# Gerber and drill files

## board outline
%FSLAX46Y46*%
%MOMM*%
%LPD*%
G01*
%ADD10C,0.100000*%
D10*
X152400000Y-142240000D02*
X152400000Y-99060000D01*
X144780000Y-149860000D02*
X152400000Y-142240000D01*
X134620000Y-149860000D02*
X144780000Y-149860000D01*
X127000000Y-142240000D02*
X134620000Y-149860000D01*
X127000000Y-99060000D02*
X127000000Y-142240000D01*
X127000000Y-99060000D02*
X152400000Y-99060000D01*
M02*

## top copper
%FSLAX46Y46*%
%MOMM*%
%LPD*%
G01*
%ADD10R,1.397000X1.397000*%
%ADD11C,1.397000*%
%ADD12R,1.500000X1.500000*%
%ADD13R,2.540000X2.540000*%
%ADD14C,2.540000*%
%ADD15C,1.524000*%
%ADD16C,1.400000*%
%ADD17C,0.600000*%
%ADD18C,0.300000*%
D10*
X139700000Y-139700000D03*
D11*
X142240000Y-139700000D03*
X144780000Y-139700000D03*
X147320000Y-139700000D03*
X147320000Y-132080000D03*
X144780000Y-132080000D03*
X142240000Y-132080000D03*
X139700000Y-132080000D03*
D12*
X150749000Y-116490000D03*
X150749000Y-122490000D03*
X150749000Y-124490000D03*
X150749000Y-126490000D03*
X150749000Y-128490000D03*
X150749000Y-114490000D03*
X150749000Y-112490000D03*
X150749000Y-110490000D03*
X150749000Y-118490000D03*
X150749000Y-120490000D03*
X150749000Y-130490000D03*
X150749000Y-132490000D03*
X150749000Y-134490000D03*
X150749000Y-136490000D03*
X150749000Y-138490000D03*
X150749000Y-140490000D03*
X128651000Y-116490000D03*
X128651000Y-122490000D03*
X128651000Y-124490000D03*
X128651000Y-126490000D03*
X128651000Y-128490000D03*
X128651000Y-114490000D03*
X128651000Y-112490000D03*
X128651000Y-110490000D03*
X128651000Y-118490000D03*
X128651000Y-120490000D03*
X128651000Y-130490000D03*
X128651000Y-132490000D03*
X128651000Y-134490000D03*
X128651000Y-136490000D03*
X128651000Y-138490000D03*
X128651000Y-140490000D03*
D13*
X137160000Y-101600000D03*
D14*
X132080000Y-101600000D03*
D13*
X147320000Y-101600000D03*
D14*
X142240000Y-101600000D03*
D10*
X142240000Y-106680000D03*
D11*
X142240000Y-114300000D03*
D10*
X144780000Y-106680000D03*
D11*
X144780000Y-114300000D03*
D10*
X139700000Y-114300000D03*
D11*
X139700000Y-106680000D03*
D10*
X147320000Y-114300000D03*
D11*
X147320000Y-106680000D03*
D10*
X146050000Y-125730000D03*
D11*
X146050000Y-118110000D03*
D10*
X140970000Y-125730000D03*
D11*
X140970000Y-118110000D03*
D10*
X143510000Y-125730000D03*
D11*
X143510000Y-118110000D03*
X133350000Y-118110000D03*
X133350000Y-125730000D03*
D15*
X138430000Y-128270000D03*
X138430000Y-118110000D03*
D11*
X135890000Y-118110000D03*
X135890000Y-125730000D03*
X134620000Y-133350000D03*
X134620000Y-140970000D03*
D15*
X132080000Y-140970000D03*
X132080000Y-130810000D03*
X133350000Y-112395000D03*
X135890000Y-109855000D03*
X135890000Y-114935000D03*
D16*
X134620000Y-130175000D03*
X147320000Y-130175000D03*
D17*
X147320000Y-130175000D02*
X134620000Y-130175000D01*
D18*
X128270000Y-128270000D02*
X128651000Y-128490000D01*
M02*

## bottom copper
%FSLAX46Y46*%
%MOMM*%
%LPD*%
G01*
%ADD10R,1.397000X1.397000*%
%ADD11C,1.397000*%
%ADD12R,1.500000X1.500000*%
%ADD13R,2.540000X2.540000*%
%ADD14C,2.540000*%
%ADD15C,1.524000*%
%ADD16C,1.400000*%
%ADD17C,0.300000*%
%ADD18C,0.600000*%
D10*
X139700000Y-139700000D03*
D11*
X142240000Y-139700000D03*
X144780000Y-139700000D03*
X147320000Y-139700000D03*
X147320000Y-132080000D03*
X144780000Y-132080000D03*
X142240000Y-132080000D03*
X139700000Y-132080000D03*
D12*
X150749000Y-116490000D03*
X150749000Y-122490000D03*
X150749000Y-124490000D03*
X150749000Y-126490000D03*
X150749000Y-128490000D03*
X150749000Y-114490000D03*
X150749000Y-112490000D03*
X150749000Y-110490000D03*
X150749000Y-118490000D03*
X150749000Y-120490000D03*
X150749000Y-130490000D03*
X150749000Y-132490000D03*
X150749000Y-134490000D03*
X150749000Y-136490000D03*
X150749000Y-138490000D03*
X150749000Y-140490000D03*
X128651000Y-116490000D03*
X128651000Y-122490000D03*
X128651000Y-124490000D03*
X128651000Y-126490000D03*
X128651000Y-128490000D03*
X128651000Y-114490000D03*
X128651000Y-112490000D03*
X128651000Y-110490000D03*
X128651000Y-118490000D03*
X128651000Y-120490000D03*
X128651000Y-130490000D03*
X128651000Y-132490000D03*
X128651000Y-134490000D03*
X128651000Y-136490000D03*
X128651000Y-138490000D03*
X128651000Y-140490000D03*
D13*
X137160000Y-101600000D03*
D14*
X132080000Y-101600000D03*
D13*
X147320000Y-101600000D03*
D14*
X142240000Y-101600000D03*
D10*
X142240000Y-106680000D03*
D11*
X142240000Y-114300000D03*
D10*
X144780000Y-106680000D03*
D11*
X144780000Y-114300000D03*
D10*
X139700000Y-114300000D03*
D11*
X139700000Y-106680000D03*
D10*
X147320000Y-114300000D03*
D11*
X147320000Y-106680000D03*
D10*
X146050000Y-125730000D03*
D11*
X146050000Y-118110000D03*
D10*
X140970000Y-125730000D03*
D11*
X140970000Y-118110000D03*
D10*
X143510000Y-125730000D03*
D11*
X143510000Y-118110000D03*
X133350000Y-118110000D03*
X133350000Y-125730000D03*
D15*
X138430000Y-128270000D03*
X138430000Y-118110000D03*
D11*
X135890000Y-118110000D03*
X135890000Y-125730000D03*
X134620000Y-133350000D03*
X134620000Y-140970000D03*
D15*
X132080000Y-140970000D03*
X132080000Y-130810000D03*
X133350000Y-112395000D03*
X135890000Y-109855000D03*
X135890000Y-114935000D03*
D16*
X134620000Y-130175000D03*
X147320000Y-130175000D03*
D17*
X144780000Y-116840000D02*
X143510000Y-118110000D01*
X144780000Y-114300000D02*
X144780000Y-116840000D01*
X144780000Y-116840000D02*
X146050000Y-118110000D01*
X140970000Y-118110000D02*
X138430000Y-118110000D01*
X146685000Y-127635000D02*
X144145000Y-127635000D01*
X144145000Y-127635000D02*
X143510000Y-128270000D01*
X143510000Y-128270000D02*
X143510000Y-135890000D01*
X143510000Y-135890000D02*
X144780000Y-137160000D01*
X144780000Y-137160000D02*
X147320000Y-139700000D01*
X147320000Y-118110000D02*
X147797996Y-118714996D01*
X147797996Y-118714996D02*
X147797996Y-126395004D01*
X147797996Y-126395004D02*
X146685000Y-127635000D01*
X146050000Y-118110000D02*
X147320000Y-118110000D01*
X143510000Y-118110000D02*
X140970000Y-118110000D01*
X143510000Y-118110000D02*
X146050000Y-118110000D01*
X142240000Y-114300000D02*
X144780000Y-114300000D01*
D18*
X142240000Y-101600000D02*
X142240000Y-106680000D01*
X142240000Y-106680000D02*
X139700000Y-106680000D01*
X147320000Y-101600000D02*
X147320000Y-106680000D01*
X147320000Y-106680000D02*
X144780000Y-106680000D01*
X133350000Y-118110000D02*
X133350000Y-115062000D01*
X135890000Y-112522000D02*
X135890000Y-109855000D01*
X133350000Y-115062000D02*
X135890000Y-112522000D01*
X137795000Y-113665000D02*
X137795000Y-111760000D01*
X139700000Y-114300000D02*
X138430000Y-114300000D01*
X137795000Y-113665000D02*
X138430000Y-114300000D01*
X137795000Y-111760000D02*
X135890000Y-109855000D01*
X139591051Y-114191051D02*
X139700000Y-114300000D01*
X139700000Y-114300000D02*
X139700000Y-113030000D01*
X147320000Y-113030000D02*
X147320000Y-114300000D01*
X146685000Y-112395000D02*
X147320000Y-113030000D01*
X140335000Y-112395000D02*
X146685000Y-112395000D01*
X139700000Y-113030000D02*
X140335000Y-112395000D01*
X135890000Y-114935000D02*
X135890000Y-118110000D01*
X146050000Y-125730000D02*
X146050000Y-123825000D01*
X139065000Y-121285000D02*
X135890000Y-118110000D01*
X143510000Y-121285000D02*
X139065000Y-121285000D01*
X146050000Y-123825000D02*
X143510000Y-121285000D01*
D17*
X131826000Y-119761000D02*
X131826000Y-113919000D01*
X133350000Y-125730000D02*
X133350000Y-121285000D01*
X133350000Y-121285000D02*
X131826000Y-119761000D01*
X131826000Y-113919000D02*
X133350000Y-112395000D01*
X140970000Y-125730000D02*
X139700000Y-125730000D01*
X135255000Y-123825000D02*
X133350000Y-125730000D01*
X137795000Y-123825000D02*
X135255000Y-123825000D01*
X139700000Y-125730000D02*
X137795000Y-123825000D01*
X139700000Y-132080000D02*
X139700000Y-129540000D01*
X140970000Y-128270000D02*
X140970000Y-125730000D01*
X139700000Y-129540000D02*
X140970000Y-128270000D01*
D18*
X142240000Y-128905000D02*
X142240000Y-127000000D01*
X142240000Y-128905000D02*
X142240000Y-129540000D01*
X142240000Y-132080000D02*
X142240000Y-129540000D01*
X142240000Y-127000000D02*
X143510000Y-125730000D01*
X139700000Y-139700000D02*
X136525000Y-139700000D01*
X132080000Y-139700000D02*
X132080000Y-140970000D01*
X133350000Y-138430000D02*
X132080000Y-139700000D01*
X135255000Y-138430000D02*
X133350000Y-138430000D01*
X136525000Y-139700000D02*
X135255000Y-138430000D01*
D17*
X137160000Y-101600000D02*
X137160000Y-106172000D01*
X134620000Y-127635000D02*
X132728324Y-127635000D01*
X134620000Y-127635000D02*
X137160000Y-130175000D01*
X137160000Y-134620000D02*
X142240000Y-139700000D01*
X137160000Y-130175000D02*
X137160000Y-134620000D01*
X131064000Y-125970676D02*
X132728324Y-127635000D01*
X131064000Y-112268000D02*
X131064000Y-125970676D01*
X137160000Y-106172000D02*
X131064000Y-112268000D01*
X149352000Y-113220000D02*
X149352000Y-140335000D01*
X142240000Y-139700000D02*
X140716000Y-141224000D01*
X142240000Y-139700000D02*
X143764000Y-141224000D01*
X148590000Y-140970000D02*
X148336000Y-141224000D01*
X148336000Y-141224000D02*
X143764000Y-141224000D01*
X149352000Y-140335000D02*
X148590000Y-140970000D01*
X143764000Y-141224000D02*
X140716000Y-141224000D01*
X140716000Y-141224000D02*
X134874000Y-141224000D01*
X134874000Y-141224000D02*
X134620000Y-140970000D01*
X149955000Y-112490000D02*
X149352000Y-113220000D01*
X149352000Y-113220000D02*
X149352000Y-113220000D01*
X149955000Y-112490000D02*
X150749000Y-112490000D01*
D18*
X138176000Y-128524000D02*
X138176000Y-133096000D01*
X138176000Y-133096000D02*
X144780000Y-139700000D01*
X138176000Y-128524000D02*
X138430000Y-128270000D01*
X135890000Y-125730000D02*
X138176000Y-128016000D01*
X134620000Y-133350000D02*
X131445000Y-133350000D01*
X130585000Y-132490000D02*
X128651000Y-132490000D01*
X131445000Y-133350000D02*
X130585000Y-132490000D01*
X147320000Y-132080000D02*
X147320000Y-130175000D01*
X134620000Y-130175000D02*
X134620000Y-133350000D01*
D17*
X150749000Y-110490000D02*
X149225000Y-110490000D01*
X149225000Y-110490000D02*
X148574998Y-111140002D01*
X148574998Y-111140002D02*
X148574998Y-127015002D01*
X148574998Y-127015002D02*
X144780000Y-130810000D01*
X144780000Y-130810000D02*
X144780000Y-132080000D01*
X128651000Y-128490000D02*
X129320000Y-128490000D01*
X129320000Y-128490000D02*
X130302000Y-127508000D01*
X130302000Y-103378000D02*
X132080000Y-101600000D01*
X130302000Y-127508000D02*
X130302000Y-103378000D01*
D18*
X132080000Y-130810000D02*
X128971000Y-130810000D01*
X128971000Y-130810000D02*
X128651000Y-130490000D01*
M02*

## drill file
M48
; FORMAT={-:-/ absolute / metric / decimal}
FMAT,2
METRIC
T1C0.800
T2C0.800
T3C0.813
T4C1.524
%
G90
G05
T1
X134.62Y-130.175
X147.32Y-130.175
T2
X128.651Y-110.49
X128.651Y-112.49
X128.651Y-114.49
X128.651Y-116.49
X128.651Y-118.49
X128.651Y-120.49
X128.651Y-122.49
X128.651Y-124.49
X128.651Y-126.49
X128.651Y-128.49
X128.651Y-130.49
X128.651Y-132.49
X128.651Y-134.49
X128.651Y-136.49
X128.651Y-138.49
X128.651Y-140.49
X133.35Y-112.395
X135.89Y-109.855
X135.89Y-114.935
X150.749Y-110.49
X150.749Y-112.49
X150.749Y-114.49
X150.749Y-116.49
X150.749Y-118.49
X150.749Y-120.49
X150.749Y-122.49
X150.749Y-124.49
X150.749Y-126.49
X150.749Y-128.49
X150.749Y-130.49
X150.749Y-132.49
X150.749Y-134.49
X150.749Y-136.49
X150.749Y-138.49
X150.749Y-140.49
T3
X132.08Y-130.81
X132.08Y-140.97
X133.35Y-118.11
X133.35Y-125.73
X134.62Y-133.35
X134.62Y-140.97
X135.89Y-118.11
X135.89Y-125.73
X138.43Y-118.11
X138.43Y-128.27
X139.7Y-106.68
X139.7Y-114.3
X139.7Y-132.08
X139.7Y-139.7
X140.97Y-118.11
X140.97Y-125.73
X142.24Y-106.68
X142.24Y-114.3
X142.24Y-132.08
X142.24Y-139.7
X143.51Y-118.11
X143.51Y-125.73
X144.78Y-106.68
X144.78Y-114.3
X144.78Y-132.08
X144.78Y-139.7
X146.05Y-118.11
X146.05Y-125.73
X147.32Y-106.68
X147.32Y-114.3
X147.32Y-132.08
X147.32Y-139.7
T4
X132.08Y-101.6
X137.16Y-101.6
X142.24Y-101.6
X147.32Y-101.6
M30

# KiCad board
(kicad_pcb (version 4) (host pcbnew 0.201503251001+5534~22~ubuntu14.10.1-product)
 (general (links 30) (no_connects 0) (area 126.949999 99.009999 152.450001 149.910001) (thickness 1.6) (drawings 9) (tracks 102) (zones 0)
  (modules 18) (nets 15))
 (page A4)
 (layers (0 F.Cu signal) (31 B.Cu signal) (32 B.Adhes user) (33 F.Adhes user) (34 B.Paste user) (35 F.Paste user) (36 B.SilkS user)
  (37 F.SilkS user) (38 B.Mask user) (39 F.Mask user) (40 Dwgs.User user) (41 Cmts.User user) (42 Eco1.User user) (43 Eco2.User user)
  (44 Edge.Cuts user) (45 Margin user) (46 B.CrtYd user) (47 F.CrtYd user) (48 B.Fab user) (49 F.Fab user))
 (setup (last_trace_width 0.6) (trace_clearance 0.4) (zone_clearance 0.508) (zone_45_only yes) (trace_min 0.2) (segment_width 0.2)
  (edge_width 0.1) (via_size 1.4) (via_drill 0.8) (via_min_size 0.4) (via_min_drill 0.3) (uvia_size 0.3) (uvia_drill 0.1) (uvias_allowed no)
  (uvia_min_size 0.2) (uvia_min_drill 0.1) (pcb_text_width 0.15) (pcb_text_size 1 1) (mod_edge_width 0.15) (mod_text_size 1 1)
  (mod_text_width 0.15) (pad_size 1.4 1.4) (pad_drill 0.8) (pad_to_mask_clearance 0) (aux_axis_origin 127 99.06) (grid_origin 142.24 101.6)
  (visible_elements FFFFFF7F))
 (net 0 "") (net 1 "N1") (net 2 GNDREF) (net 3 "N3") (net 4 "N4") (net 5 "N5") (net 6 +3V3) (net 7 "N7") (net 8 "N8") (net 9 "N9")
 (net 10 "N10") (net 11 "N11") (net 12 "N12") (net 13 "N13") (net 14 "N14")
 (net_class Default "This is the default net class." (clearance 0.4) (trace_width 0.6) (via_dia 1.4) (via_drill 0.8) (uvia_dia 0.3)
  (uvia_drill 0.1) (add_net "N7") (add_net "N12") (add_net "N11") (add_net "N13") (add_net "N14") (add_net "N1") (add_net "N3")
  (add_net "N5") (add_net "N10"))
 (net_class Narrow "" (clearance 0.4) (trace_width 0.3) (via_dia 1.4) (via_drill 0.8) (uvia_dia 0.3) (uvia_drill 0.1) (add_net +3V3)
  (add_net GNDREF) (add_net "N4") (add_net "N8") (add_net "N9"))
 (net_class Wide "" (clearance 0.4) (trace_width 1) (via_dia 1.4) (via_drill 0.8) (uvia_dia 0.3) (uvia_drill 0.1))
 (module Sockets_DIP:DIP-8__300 (layer F.Cu) (at 143.51 135.89)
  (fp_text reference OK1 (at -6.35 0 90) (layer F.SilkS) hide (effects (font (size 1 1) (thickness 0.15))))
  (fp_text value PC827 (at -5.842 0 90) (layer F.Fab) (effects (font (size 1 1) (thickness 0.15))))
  (pad 1 thru_hole rect (at -3.81 3.81) (size 1.397 1.397) (drill 0.8128) (layers *.Cu *.Mask F.SilkS) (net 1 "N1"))
  (pad 2 thru_hole circle (at -1.27 3.81) (size 1.397 1.397) (drill 0.8128) (layers *.Cu *.Mask F.SilkS) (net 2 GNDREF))
  (pad 3 thru_hole circle (at 1.27 3.81) (size 1.397 1.397) (drill 0.8128) (layers *.Cu *.Mask F.SilkS) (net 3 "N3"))
  (pad 4 thru_hole circle (at 3.81 3.81) (size 1.397 1.397) (drill 0.8128) (layers *.Cu *.Mask F.SilkS) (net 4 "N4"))
  (pad 5 thru_hole circle (at 3.81 -3.81) (size 1.397 1.397) (drill 0.8128) (layers *.Cu *.Mask F.SilkS) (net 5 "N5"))
  (pad 6 thru_hole circle (at 1.27 -3.81) (size 1.397 1.397) (drill 0.8128) (layers *.Cu *.Mask F.SilkS) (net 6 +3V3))
  (pad 7 thru_hole circle (at -1.27 -3.81) (size 1.397 1.397) (drill 0.8128) (layers *.Cu *.Mask F.SilkS) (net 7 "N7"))
  (pad 8 thru_hole circle (at -3.81 -3.81) (size 1.397 1.397) (drill 0.8128) (layers *.Cu *.Mask F.SilkS) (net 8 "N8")))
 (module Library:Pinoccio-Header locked (layer F.Cu) (at 150.749 125.49)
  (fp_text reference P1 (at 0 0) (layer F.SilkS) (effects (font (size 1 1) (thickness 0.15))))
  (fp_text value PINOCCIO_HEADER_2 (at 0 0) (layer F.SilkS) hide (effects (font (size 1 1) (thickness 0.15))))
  (pad 4 thru_hole rect (at 0 -9) (size 1.5 1.5) (drill 0.8) (layers *.Cu *.Mask F.SilkS))
  (pad 7 thru_hole rect (at 0 -3) (size 1.5 1.5) (drill 0.8) (layers *.Cu *.Mask F.SilkS))
  (pad 8 thru_hole rect (at 0 -1) (size 1.5 1.5) (drill 0.8) (layers *.Cu *.Mask F.SilkS))
  (pad 9 thru_hole rect (at 0 1) (size 1.5 1.5) (drill 0.8) (layers *.Cu *.Mask F.SilkS))
  (pad 10 thru_hole rect (at 0 3) (size 1.5 1.5) (drill 0.8) (layers *.Cu *.Mask F.SilkS))
  (pad 3 thru_hole rect (at 0 -11) (size 1.5 1.5) (drill 0.8) (layers *.Cu *.Mask F.SilkS))
  (pad 2 thru_hole rect (at 0 -13) (size 1.5 1.5) (drill 0.8) (layers *.Cu *.Mask F.SilkS) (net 2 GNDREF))
  (pad 1 thru_hole rect (at 0 -15) (size 1.5 1.5) (drill 0.8) (layers *.Cu *.Mask F.SilkS) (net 6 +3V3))
  (pad 5 thru_hole rect (at 0 -7) (size 1.5 1.5) (drill 0.8) (layers *.Cu *.Mask F.SilkS))
  (pad 6 thru_hole rect (at 0 -5) (size 1.5 1.5) (drill 0.8) (layers *.Cu *.Mask F.SilkS))
  (pad 11 thru_hole rect (at 0 5) (size 1.5 1.5) (drill 0.8) (layers *.Cu *.Mask F.SilkS))
  (pad 12 thru_hole rect (at 0 7) (size 1.5 1.5) (drill 0.8) (layers *.Cu *.Mask F.SilkS))
  (pad 13 thru_hole rect (at 0 9) (size 1.5 1.5) (drill 0.8) (layers *.Cu *.Mask F.SilkS))
  (pad 14 thru_hole rect (at 0 11) (size 1.5 1.5) (drill 0.8) (layers *.Cu *.Mask F.SilkS))
  (pad 15 thru_hole rect (at 0 13) (size 1.5 1.5) (drill 0.8) (layers *.Cu *.Mask F.SilkS))
  (pad 16 thru_hole rect (at 0 15) (size 1.5 1.5) (drill 0.8) (layers *.Cu *.Mask F.SilkS)))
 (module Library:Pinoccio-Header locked (layer F.Cu) (at 128.651 125.49)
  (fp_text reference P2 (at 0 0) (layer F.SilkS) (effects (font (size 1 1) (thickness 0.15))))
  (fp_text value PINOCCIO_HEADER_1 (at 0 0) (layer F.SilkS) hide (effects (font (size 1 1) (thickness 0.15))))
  (pad 4 thru_hole rect (at 0 -9) (size 1.5 1.5) (drill 0.8) (layers *.Cu *.Mask F.SilkS))
  (pad 7 thru_hole rect (at 0 -3) (size 1.5 1.5) (drill 0.8) (layers *.Cu *.Mask F.SilkS))
  (pad 8 thru_hole rect (at 0 -1) (size 1.5 1.5) (drill 0.8) (layers *.Cu *.Mask F.SilkS))
  (pad 9 thru_hole rect (at 0 1) (size 1.5 1.5) (drill 0.8) (layers *.Cu *.Mask F.SilkS))
  (pad 10 thru_hole rect (at 0 3) (size 1.5 1.5) (drill 0.8) (layers *.Cu *.Mask F.SilkS) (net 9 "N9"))
  (pad 3 thru_hole rect (at 0 -11) (size 1.5 1.5) (drill 0.8) (layers *.Cu *.Mask F.SilkS))
  (pad 2 thru_hole rect (at 0 -13) (size 1.5 1.5) (drill 0.8) (layers *.Cu *.Mask F.SilkS))
  (pad 1 thru_hole rect (at 0 -15) (size 1.5 1.5) (drill 0.8) (layers *.Cu *.Mask F.SilkS))
  (pad 5 thru_hole rect (at 0 -7) (size 1.5 1.5) (drill 0.8) (layers *.Cu *.Mask F.SilkS))
  (pad 6 thru_hole rect (at 0 -5) (size 1.5 1.5) (drill 0.8) (layers *.Cu *.Mask F.SilkS))
  (pad 11 thru_hole rect (at 0 5) (size 1.5 1.5) (drill 0.8) (layers *.Cu *.Mask F.SilkS) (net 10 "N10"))
  (pad 12 thru_hole rect (at 0 7) (size 1.5 1.5) (drill 0.8) (layers *.Cu *.Mask F.SilkS) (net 5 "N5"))
  (pad 13 thru_hole rect (at 0 9) (size 1.5 1.5) (drill 0.8) (layers *.Cu *.Mask F.SilkS))
  (pad 14 thru_hole rect (at 0 11) (size 1.5 1.5) (drill 0.8) (layers *.Cu *.Mask F.SilkS))
  (pad 15 thru_hole rect (at 0 13) (size 1.5 1.5) (drill 0.8) (layers *.Cu *.Mask F.SilkS))
  (pad 16 thru_hole rect (at 0 15) (size 1.5 1.5) (drill 0.8) (layers *.Cu *.Mask F.SilkS)))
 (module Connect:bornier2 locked (layer F.Cu) (at 134.62 101.6 180)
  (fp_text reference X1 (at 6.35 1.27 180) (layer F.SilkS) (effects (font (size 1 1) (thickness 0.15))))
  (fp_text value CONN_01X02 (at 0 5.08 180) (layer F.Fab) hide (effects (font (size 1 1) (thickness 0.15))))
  (pad 1 thru_hole rect (at -2.54 0 180) (size 2.54 2.54) (drill 1.524) (layers *.Cu *.Mask F.SilkS) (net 2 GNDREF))
  (pad 2 thru_hole circle (at 2.54 0 180) (size 2.54 2.54) (drill 1.524) (layers *.Cu *.Mask F.SilkS) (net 9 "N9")))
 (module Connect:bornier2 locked (layer F.Cu) (at 144.78 101.6 180)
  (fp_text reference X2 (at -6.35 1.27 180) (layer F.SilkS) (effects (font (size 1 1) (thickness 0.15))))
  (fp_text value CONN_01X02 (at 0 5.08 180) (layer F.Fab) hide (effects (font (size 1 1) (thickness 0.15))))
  (pad 1 thru_hole rect (at -2.54 0 180) (size 2.54 2.54) (drill 1.524) (layers *.Cu *.Mask F.SilkS) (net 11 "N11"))
  (pad 2 thru_hole circle (at 2.54 0 180) (size 2.54 2.54) (drill 1.524) (layers *.Cu *.Mask F.SilkS) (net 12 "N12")))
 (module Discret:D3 (layer F.Cu) (at 142.24 110.49 90)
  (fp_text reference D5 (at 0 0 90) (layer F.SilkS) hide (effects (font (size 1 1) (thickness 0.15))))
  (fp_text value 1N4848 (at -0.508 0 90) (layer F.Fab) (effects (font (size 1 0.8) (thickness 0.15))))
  (pad 2 thru_hole rect (at 3.81 0 90) (size 1.397 1.397) (drill 0.8128) (layers *.Cu *.Mask F.SilkS) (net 12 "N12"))
  (pad 1 thru_hole circle (at -3.81 0 90) (size 1.397 1.397) (drill 0.8128) (layers *.Cu *.Mask F.SilkS) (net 4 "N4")))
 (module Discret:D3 (layer F.Cu) (at 144.78 110.49 90)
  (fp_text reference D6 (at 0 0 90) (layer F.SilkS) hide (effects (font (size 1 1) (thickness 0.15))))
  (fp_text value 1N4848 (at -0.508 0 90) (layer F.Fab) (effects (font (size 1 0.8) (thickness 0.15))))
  (pad 2 thru_hole rect (at 3.81 0 90) (size 1.397 1.397) (drill 0.8128) (layers *.Cu *.Mask F.SilkS) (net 11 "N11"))
  (pad 1 thru_hole circle (at -3.81 0 90) (size 1.397 1.397) (drill 0.8128) (layers *.Cu *.Mask F.SilkS) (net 4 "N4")))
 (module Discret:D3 (layer F.Cu) (at 139.7 110.49 270)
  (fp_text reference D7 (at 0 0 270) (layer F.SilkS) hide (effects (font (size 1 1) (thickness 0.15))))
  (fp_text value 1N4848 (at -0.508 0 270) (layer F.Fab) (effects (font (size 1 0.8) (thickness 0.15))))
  (pad 2 thru_hole rect (at 3.81 0 270) (size 1.397 1.397) (drill 0.8128) (layers *.Cu *.Mask F.SilkS) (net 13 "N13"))
  (pad 1 thru_hole circle (at -3.81 0 270) (size 1.397 1.397) (drill 0.8128) (layers *.Cu *.Mask F.SilkS) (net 12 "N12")))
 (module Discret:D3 (layer F.Cu) (at 147.32 110.49 270)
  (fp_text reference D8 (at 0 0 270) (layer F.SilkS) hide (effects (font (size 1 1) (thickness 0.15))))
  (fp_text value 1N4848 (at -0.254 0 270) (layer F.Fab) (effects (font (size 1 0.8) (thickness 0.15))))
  (pad 2 thru_hole rect (at 3.81 0 270) (size 1.397 1.397) (drill 0.8128) (layers *.Cu *.Mask F.SilkS) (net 13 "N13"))
  (pad 1 thru_hole circle (at -3.81 0 270) (size 1.397 1.397) (drill 0.8128) (layers *.Cu *.Mask F.SilkS) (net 11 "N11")))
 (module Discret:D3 (layer F.Cu) (at 146.05 121.92 270)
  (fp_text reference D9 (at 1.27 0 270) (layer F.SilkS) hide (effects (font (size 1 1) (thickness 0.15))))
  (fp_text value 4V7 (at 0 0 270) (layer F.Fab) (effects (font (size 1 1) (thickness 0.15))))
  (pad 2 thru_hole rect (at 3.81 0 270) (size 1.397 1.397) (drill 0.8128) (layers *.Cu *.Mask F.SilkS) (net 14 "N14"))
  (pad 1 thru_hole circle (at -3.81 0 270) (size 1.397 1.397) (drill 0.8128) (layers *.Cu *.Mask F.SilkS) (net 4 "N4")))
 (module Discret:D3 (layer F.Cu) (at 140.97 121.92 270)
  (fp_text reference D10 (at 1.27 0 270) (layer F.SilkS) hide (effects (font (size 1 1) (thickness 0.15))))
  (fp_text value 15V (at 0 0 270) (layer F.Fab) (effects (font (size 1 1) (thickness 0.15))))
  (pad 2 thru_hole rect (at 3.81 0 270) (size 1.397 1.397) (drill 0.8128) (layers *.Cu *.Mask F.SilkS) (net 8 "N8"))
  (pad 1 thru_hole circle (at -3.81 0 270) (size 1.397 1.397) (drill 0.8128) (layers *.Cu *.Mask F.SilkS) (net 4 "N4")))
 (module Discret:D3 (layer F.Cu) (at 143.51 121.92 270)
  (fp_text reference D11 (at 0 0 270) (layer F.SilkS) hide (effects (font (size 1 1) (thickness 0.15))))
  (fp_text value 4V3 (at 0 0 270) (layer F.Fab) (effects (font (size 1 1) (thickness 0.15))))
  (pad 2 thru_hole rect (at 3.81 0 270) (size 1.397 1.397) (drill 0.8128) (layers *.Cu *.Mask F.SilkS) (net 7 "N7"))
  (pad 1 thru_hole circle (at -3.81 0 270) (size 1.397 1.397) (drill 0.8128) (layers *.Cu *.Mask F.SilkS) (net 4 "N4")))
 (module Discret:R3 (layer F.Cu) (at 133.35 121.92 270)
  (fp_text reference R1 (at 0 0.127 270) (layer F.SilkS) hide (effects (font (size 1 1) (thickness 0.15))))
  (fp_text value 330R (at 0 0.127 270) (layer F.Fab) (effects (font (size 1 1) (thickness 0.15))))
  (pad 1 thru_hole circle (at -3.81 0 270) (size 1.397 1.397) (drill 0.8128) (layers *.Cu *.Mask F.SilkS) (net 13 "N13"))
  (pad 2 thru_hole circle (at 3.81 0 270) (size 1.397 1.397) (drill 0.8128) (layers *.Cu *.Mask F.SilkS) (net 8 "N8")))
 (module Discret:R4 (layer F.Cu) (at 138.43 123.19 90)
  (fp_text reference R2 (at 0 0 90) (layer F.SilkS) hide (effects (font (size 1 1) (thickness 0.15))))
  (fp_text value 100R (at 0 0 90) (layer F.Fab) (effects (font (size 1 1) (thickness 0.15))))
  (pad 1 thru_hole circle (at -5.08 0 90) (size 1.524 1.524) (drill 0.8128) (layers *.Cu *.Mask F.SilkS) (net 3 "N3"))
  (pad 2 thru_hole circle (at 5.08 0 90) (size 1.524 1.524) (drill 0.8128) (layers *.Cu *.Mask F.SilkS) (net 4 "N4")))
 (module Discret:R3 (layer F.Cu) (at 135.89 121.92 270)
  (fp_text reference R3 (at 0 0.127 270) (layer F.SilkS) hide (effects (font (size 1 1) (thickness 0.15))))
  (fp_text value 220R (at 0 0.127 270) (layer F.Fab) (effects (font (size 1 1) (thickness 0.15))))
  (pad 1 thru_hole circle (at -3.81 0 270) (size 1.397 1.397) (drill 0.8128) (layers *.Cu *.Mask F.SilkS) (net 14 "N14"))
  (pad 2 thru_hole circle (at 3.81 0 270) (size 1.397 1.397) (drill 0.8128) (layers *.Cu *.Mask F.SilkS) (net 3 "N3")))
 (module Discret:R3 (layer F.Cu) (at 134.62 137.16 270)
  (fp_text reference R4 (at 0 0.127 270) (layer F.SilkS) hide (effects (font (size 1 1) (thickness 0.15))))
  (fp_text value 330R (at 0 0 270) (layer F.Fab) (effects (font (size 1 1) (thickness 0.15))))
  (pad 1 thru_hole circle (at -3.81 0 270) (size 1.397 1.397) (drill 0.8128) (layers *.Cu *.Mask F.SilkS) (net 5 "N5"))
  (pad 2 thru_hole circle (at 3.81 0 270) (size 1.397 1.397) (drill 0.8128) (layers *.Cu *.Mask F.SilkS) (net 2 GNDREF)))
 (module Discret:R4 (layer F.Cu) (at 132.08 135.89 90)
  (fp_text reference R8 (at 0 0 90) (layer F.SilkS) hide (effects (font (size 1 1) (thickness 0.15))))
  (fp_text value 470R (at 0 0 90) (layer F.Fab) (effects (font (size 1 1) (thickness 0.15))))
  (pad 1 thru_hole circle (at -5.08 0 90) (size 1.524 1.524) (drill 0.8128) (layers *.Cu *.Mask F.SilkS) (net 1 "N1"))
  (pad 2 thru_hole circle (at 5.08 0 90) (size 1.524 1.524) (drill 0.8128) (layers *.Cu *.Mask F.SilkS) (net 10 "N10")))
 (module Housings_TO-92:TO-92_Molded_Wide (layer F.Cu) (at 135.89 114.935 90)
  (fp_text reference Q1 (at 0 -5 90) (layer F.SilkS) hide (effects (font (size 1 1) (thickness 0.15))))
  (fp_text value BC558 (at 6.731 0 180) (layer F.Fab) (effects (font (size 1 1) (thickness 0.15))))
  (pad 2 thru_hole circle (at 2.54 -2.54 180) (size 1.524 1.524) (drill 0.8) (layers *.Cu *.Mask F.SilkS) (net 8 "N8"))
  (pad 3 thru_hole circle (at 5.08 0 180) (size 1.524 1.524) (drill 0.8) (layers *.Cu *.Mask F.SilkS) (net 13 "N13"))
  (pad 1 thru_hole circle (at 0 0 180) (size 1.524 1.524) (drill 0.8) (layers *.Cu *.Mask F.SilkS) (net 14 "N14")))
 (gr_line (start 152.4 142.24) (end 152.4 99.06) (angle 90) (layer Edge.Cuts) (width 0.1))
 (gr_line (start 144.78 149.86) (end 152.4 142.24) (angle 90) (layer Edge.Cuts) (width 0.1))
 (gr_line (start 134.62 149.86) (end 144.78 149.86) (angle 90) (layer Edge.Cuts) (width 0.1))
 (gr_line (start 127 142.24) (end 134.62 149.86) (angle 90) (layer Edge.Cuts) (width 0.1))
 (gr_line (start 127 99.06) (end 127 142.24) (angle 90) (layer Edge.Cuts) (width 0.1))
 (gr_line (start 127 99.06) (end 152.4 99.06) (angle 90) (layer Edge.Cuts) (width 0.1))
 (segment (start 144.78 116.84) (end 143.51 118.11) (width 0.3) (layer B.Cu) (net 4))
 (segment (start 144.78 114.3) (end 144.78 116.84) (width 0.3) (layer B.Cu) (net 4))
 (segment (start 144.78 116.84) (end 146.05 118.11) (width 0.3) (layer B.Cu) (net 4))
 (segment (start 140.97 118.11) (end 138.43 118.11) (width 0.3) (layer B.Cu) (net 4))
 (segment (start 146.685 127.635) (end 144.145 127.635) (width 0.3) (layer B.Cu) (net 4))
 (segment (start 144.145 127.635) (end 143.51 128.27) (width 0.3) (layer B.Cu) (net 4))
 (segment (start 143.51 128.27) (end 143.51 135.89) (width 0.3) (layer B.Cu) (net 4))
 (segment (start 143.51 135.89) (end 144.78 137.16) (width 0.3) (layer B.Cu) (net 4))
 (segment (start 144.78 137.16) (end 147.32 139.7) (width 0.3) (layer B.Cu) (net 4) (status 20))
 (segment (start 147.32 118.11) (end 147.797996 118.714996) (width 0.3) (layer B.Cu) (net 4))
 (segment (start 147.797996 118.714996) (end 147.797996 126.395004) (width 0.3) (layer B.Cu) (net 4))
 (segment (start 147.797996 126.395004) (end 146.685 127.635) (width 0.3) (layer B.Cu) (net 4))
 (segment (start 146.05 118.11) (end 147.32 118.11) (width 0.3) (layer B.Cu) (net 4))
 (segment (start 143.51 118.11) (end 140.97 118.11) (width 0.3) (layer B.Cu) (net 4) (status 80010))
 (segment (start 143.51 118.11) (end 146.05 118.11) (width 0.3) (layer B.Cu) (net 4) (status 80020))
 (segment (start 142.24 114.3) (end 144.78 114.3) (width 0.3) (layer B.Cu) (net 4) (status 80020))
 (segment (start 142.24 101.6) (end 142.24 106.68) (width 0.6) (layer B.Cu) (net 12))
 (segment (start 142.24 106.68) (end 139.7 106.68) (width 0.6) (layer B.Cu) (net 12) (status 80010))
 (segment (start 147.32 101.6) (end 147.32 106.68) (width 0.6) (layer B.Cu) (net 11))
 (segment (start 147.32 106.68) (end 144.78 106.68) (width 0.6) (layer B.Cu) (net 11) (status 80010))
 (segment (start 133.35 118.11) (end 133.35 115.062) (width 0.6) (layer B.Cu) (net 13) (status 400000))
 (segment (start 135.89 112.522) (end 135.89 109.855) (width 0.6) (layer B.Cu) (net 13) (status 800000))
 (segment (start 133.35 115.062) (end 135.89 112.522) (width 0.6) (layer B.Cu) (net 13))
 (segment (start 137.795 113.665) (end 137.795 111.76) (width 0.6) (layer B.Cu) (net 13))
 (segment (start 139.7 114.3) (end 138.43 114.3) (width 0.6) (layer B.Cu) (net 13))
 (segment (start 137.795 113.665) (end 138.43 114.3) (width 0.6) (layer B.Cu) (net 13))
 (segment (start 137.795 111.76) (end 135.89 109.855) (width 0.6) (layer B.Cu) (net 13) (status 800000))
 (segment (start 139.591051 114.191051) (end 139.7 114.3) (width 0.6) (layer B.Cu) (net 13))
 (segment (start 139.7 114.3) (end 139.7 113.03) (width 0.6) (layer B.Cu) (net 13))
 (segment (start 147.32 113.03) (end 147.32 114.3) (width 0.6) (layer B.Cu) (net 13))
 (segment (start 146.685 112.395) (end 147.32 113.03) (width 0.6) (layer B.Cu) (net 13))
 (segment (start 140.335 112.395) (end 146.685 112.395) (width 0.6) (layer B.Cu) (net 13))
 (segment (start 139.7 113.03) (end 140.335 112.395) (width 0.6) (layer B.Cu) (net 13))
 (segment (start 135.89 114.935) (end 135.89 118.11) (width 0.6) (layer B.Cu) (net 14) (status C00000))
 (segment (start 146.05 125.73) (end 146.05 123.825) (width 0.6) (layer B.Cu) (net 14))
 (segment (start 139.065 121.285) (end 135.89 118.11) (width 0.6) (layer B.Cu) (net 14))
 (segment (start 143.51 121.285) (end 139.065 121.285) (width 0.6) (layer B.Cu) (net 14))
 (segment (start 146.05 123.825) (end 143.51 121.285) (width 0.6) (layer B.Cu) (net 14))
 (segment (start 131.826 119.761) (end 131.826 113.919) (width 0.3) (layer B.Cu) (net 8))
 (segment (start 133.35 125.73) (end 133.35 121.285) (width 0.3) (layer B.Cu) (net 8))
 (segment (start 133.35 121.285) (end 131.826 119.761) (width 0.3) (layer B.Cu) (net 8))
 (segment (start 131.826 113.919) (end 133.35 112.395) (width 0.3) (layer B.Cu) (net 8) (status 800000))
 (segment (start 140.97 125.73) (end 139.7 125.73) (width 0.3) (layer B.Cu) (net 8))
 (segment (start 135.255 123.825) (end 133.35 125.73) (width 0.3) (layer B.Cu) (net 8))
 (segment (start 137.795 123.825) (end 135.255 123.825) (width 0.3) (layer B.Cu) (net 8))
 (segment (start 139.7 125.73) (end 137.795 123.825) (width 0.3) (layer B.Cu) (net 8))
 (segment (start 139.7 132.08) (end 139.7 129.54) (width 0.3) (layer B.Cu) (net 8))
 (segment (start 140.97 128.27) (end 140.97 125.73) (width 0.3) (layer B.Cu) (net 8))
 (segment (start 139.7 129.54) (end 140.97 128.27) (width 0.3) (layer B.Cu) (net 8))
 (segment (start 142.24 128.905) (end 142.24 127) (width 0.6) (layer B.Cu) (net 7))
 (segment (start 142.24 128.905) (end 142.24 129.54) (width 0.6) (layer B.Cu) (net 7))
 (segment (start 142.24 132.08) (end 142.24 129.54) (width 0.6) (layer B.Cu) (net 7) (status 20))
 (segment (start 142.24 127) (end 143.51 125.73) (width 0.6) (layer B.Cu) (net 7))
 (segment (start 139.7 139.7) (end 136.525 139.7) (width 0.6) (layer B.Cu) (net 1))
 (segment (start 132.08 139.7) (end 132.08 140.97) (width 0.6) (layer B.Cu) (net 1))
 (segment (start 133.35 138.43) (end 132.08 139.7) (width 0.6) (layer B.Cu) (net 1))
 (segment (start 135.255 138.43) (end 133.35 138.43) (width 0.6) (layer B.Cu) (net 1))
 (segment (start 136.525 139.7) (end 135.255 138.43) (width 0.6) (layer B.Cu) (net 1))
 (segment (start 137.16 101.6) (end 137.16 106.172) (width 0.3) (layer B.Cu) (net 2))
 (segment (start 134.62 127.635) (end 132.728324 127.635) (width 0.3) (layer B.Cu) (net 2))
 (segment (start 134.62 127.635) (end 137.16 130.175) (width 0.3) (layer B.Cu) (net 2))
 (segment (start 137.16 134.62) (end 142.24 139.7) (width 0.3) (layer B.Cu) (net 2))
 (segment (start 137.16 130.175) (end 137.16 134.62) (width 0.3) (layer B.Cu) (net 2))
 (segment (start 131.064 125.970676) (end 132.728324 127.635) (width 0.3) (layer B.Cu) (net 2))
 (segment (start 131.064 112.268) (end 131.064 125.970676) (width 0.3) (layer B.Cu) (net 2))
 (segment (start 137.16 106.172) (end 131.064 112.268) (width 0.3) (layer B.Cu) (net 2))
 (segment (start 149.352 113.22) (end 149.352 140.335) (width 0.3) (layer B.Cu) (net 2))
 (segment (start 142.24 139.7) (end 140.716 141.224) (width 0.3) (layer B.Cu) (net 2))
 (segment (start 142.24 139.7) (end 143.764 141.224) (width 0.3) (layer B.Cu) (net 2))
 (segment (start 148.59 140.97) (end 148.336 141.224) (width 0.3) (layer B.Cu) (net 2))
 (segment (start 148.336 141.224) (end 143.764 141.224) (width 0.3) (layer B.Cu) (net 2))
 (segment (start 149.352 140.335) (end 148.59 140.97) (width 0.3) (layer B.Cu) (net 2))
 (segment (start 143.764 141.224) (end 140.716 141.224) (width 0.3) (layer B.Cu) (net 2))
 (segment (start 140.716 141.224) (end 134.874 141.224) (width 0.3) (layer B.Cu) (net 2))
 (segment (start 134.874 141.224) (end 134.62 140.97) (width 0.3) (layer B.Cu) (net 2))
 (segment (start 149.955 112.49) (end 149.352 113.22) (width 0.3) (layer B.Cu) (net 2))
 (segment (start 149.352 113.22) (end 149.352 113.22) (width 0.3) (layer B.Cu) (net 2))
 (segment (start 149.955 112.49) (end 150.749 112.49) (width 0.3) (layer B.Cu) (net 2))
 (segment (start 138.176 128.524) (end 138.176 133.096) (width 0.6) (layer B.Cu) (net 3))
 (segment (start 138.176 133.096) (end 144.78 139.7) (width 0.6) (layer B.Cu) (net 3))
 (segment (start 138.176 128.524) (end 138.43 128.27) (width 0.6) (layer B.Cu) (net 3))
 (segment (start 135.89 125.73) (end 138.176 128.016) (width 0.6) (layer B.Cu) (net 3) (status 80020))
 (segment (start 134.62 133.35) (end 131.445 133.35) (width 0.6) (layer B.Cu) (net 5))
 (segment (start 130.585 132.49) (end 128.651 132.49) (width 0.6) (layer B.Cu) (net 5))
 (segment (start 131.445 133.35) (end 130.585 132.49) (width 0.6) (layer B.Cu) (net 5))
 (segment (start 147.32 132.08) (end 147.32 130.175) (width 0.6) (layer B.Cu) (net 5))
 (segment (start 134.62 130.175) (end 134.62 133.35) (width 0.6) (layer B.Cu) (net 5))
 (via (at 134.62 130.175) (size 1.4) (layers F.Cu B.Cu) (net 5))
 (segment (start 147.32 130.175) (end 134.62 130.175) (width 0.6) (layer F.Cu) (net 5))
 (via (at 147.32 130.175) (size 1.4) (layers F.Cu B.Cu) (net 5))
 (segment (start 150.749 110.49) (end 149.225 110.49) (width 0.3) (layer B.Cu) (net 6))
 (segment (start 149.225 110.49) (end 148.574998 111.140002) (width 0.3) (layer B.Cu) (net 6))
 (segment (start 148.574998 111.140002) (end 148.574998 127.015002) (width 0.3) (layer B.Cu) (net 6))
 (segment (start 148.574998 127.015002) (end 144.78 130.81) (width 0.3) (layer B.Cu) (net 6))
 (segment (start 144.78 130.81) (end 144.78 132.08) (width 0.3) (layer B.Cu) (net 6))
 (segment (start 128.651 128.49) (end 129.32 128.49) (width 0.3) (layer B.Cu) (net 9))
 (segment (start 129.32 128.49) (end 130.302 127.508) (width 0.3) (layer B.Cu) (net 9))
 (segment (start 130.302 103.378) (end 132.08 101.6) (width 0.3) (layer B.Cu) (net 9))
 (segment (start 130.302 127.508) (end 130.302 103.378) (width 0.3) (layer B.Cu) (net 9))
 (segment (start 128.27 128.27) (end 128.651 128.49) (width 0.3) (layer F.Cu) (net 9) (status 80000))
 (segment (start 132.08 130.81) (end 128.971 130.81) (width 0.6) (layer B.Cu) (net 10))
 (segment (start 128.971 130.81) (end 128.651 130.49) (width 0.6) (layer B.Cu) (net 10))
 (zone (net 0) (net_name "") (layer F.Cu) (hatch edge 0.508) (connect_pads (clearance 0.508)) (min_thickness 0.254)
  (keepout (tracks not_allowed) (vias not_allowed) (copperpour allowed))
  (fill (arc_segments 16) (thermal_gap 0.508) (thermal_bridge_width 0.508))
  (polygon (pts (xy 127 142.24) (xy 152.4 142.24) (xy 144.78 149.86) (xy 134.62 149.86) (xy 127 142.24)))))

